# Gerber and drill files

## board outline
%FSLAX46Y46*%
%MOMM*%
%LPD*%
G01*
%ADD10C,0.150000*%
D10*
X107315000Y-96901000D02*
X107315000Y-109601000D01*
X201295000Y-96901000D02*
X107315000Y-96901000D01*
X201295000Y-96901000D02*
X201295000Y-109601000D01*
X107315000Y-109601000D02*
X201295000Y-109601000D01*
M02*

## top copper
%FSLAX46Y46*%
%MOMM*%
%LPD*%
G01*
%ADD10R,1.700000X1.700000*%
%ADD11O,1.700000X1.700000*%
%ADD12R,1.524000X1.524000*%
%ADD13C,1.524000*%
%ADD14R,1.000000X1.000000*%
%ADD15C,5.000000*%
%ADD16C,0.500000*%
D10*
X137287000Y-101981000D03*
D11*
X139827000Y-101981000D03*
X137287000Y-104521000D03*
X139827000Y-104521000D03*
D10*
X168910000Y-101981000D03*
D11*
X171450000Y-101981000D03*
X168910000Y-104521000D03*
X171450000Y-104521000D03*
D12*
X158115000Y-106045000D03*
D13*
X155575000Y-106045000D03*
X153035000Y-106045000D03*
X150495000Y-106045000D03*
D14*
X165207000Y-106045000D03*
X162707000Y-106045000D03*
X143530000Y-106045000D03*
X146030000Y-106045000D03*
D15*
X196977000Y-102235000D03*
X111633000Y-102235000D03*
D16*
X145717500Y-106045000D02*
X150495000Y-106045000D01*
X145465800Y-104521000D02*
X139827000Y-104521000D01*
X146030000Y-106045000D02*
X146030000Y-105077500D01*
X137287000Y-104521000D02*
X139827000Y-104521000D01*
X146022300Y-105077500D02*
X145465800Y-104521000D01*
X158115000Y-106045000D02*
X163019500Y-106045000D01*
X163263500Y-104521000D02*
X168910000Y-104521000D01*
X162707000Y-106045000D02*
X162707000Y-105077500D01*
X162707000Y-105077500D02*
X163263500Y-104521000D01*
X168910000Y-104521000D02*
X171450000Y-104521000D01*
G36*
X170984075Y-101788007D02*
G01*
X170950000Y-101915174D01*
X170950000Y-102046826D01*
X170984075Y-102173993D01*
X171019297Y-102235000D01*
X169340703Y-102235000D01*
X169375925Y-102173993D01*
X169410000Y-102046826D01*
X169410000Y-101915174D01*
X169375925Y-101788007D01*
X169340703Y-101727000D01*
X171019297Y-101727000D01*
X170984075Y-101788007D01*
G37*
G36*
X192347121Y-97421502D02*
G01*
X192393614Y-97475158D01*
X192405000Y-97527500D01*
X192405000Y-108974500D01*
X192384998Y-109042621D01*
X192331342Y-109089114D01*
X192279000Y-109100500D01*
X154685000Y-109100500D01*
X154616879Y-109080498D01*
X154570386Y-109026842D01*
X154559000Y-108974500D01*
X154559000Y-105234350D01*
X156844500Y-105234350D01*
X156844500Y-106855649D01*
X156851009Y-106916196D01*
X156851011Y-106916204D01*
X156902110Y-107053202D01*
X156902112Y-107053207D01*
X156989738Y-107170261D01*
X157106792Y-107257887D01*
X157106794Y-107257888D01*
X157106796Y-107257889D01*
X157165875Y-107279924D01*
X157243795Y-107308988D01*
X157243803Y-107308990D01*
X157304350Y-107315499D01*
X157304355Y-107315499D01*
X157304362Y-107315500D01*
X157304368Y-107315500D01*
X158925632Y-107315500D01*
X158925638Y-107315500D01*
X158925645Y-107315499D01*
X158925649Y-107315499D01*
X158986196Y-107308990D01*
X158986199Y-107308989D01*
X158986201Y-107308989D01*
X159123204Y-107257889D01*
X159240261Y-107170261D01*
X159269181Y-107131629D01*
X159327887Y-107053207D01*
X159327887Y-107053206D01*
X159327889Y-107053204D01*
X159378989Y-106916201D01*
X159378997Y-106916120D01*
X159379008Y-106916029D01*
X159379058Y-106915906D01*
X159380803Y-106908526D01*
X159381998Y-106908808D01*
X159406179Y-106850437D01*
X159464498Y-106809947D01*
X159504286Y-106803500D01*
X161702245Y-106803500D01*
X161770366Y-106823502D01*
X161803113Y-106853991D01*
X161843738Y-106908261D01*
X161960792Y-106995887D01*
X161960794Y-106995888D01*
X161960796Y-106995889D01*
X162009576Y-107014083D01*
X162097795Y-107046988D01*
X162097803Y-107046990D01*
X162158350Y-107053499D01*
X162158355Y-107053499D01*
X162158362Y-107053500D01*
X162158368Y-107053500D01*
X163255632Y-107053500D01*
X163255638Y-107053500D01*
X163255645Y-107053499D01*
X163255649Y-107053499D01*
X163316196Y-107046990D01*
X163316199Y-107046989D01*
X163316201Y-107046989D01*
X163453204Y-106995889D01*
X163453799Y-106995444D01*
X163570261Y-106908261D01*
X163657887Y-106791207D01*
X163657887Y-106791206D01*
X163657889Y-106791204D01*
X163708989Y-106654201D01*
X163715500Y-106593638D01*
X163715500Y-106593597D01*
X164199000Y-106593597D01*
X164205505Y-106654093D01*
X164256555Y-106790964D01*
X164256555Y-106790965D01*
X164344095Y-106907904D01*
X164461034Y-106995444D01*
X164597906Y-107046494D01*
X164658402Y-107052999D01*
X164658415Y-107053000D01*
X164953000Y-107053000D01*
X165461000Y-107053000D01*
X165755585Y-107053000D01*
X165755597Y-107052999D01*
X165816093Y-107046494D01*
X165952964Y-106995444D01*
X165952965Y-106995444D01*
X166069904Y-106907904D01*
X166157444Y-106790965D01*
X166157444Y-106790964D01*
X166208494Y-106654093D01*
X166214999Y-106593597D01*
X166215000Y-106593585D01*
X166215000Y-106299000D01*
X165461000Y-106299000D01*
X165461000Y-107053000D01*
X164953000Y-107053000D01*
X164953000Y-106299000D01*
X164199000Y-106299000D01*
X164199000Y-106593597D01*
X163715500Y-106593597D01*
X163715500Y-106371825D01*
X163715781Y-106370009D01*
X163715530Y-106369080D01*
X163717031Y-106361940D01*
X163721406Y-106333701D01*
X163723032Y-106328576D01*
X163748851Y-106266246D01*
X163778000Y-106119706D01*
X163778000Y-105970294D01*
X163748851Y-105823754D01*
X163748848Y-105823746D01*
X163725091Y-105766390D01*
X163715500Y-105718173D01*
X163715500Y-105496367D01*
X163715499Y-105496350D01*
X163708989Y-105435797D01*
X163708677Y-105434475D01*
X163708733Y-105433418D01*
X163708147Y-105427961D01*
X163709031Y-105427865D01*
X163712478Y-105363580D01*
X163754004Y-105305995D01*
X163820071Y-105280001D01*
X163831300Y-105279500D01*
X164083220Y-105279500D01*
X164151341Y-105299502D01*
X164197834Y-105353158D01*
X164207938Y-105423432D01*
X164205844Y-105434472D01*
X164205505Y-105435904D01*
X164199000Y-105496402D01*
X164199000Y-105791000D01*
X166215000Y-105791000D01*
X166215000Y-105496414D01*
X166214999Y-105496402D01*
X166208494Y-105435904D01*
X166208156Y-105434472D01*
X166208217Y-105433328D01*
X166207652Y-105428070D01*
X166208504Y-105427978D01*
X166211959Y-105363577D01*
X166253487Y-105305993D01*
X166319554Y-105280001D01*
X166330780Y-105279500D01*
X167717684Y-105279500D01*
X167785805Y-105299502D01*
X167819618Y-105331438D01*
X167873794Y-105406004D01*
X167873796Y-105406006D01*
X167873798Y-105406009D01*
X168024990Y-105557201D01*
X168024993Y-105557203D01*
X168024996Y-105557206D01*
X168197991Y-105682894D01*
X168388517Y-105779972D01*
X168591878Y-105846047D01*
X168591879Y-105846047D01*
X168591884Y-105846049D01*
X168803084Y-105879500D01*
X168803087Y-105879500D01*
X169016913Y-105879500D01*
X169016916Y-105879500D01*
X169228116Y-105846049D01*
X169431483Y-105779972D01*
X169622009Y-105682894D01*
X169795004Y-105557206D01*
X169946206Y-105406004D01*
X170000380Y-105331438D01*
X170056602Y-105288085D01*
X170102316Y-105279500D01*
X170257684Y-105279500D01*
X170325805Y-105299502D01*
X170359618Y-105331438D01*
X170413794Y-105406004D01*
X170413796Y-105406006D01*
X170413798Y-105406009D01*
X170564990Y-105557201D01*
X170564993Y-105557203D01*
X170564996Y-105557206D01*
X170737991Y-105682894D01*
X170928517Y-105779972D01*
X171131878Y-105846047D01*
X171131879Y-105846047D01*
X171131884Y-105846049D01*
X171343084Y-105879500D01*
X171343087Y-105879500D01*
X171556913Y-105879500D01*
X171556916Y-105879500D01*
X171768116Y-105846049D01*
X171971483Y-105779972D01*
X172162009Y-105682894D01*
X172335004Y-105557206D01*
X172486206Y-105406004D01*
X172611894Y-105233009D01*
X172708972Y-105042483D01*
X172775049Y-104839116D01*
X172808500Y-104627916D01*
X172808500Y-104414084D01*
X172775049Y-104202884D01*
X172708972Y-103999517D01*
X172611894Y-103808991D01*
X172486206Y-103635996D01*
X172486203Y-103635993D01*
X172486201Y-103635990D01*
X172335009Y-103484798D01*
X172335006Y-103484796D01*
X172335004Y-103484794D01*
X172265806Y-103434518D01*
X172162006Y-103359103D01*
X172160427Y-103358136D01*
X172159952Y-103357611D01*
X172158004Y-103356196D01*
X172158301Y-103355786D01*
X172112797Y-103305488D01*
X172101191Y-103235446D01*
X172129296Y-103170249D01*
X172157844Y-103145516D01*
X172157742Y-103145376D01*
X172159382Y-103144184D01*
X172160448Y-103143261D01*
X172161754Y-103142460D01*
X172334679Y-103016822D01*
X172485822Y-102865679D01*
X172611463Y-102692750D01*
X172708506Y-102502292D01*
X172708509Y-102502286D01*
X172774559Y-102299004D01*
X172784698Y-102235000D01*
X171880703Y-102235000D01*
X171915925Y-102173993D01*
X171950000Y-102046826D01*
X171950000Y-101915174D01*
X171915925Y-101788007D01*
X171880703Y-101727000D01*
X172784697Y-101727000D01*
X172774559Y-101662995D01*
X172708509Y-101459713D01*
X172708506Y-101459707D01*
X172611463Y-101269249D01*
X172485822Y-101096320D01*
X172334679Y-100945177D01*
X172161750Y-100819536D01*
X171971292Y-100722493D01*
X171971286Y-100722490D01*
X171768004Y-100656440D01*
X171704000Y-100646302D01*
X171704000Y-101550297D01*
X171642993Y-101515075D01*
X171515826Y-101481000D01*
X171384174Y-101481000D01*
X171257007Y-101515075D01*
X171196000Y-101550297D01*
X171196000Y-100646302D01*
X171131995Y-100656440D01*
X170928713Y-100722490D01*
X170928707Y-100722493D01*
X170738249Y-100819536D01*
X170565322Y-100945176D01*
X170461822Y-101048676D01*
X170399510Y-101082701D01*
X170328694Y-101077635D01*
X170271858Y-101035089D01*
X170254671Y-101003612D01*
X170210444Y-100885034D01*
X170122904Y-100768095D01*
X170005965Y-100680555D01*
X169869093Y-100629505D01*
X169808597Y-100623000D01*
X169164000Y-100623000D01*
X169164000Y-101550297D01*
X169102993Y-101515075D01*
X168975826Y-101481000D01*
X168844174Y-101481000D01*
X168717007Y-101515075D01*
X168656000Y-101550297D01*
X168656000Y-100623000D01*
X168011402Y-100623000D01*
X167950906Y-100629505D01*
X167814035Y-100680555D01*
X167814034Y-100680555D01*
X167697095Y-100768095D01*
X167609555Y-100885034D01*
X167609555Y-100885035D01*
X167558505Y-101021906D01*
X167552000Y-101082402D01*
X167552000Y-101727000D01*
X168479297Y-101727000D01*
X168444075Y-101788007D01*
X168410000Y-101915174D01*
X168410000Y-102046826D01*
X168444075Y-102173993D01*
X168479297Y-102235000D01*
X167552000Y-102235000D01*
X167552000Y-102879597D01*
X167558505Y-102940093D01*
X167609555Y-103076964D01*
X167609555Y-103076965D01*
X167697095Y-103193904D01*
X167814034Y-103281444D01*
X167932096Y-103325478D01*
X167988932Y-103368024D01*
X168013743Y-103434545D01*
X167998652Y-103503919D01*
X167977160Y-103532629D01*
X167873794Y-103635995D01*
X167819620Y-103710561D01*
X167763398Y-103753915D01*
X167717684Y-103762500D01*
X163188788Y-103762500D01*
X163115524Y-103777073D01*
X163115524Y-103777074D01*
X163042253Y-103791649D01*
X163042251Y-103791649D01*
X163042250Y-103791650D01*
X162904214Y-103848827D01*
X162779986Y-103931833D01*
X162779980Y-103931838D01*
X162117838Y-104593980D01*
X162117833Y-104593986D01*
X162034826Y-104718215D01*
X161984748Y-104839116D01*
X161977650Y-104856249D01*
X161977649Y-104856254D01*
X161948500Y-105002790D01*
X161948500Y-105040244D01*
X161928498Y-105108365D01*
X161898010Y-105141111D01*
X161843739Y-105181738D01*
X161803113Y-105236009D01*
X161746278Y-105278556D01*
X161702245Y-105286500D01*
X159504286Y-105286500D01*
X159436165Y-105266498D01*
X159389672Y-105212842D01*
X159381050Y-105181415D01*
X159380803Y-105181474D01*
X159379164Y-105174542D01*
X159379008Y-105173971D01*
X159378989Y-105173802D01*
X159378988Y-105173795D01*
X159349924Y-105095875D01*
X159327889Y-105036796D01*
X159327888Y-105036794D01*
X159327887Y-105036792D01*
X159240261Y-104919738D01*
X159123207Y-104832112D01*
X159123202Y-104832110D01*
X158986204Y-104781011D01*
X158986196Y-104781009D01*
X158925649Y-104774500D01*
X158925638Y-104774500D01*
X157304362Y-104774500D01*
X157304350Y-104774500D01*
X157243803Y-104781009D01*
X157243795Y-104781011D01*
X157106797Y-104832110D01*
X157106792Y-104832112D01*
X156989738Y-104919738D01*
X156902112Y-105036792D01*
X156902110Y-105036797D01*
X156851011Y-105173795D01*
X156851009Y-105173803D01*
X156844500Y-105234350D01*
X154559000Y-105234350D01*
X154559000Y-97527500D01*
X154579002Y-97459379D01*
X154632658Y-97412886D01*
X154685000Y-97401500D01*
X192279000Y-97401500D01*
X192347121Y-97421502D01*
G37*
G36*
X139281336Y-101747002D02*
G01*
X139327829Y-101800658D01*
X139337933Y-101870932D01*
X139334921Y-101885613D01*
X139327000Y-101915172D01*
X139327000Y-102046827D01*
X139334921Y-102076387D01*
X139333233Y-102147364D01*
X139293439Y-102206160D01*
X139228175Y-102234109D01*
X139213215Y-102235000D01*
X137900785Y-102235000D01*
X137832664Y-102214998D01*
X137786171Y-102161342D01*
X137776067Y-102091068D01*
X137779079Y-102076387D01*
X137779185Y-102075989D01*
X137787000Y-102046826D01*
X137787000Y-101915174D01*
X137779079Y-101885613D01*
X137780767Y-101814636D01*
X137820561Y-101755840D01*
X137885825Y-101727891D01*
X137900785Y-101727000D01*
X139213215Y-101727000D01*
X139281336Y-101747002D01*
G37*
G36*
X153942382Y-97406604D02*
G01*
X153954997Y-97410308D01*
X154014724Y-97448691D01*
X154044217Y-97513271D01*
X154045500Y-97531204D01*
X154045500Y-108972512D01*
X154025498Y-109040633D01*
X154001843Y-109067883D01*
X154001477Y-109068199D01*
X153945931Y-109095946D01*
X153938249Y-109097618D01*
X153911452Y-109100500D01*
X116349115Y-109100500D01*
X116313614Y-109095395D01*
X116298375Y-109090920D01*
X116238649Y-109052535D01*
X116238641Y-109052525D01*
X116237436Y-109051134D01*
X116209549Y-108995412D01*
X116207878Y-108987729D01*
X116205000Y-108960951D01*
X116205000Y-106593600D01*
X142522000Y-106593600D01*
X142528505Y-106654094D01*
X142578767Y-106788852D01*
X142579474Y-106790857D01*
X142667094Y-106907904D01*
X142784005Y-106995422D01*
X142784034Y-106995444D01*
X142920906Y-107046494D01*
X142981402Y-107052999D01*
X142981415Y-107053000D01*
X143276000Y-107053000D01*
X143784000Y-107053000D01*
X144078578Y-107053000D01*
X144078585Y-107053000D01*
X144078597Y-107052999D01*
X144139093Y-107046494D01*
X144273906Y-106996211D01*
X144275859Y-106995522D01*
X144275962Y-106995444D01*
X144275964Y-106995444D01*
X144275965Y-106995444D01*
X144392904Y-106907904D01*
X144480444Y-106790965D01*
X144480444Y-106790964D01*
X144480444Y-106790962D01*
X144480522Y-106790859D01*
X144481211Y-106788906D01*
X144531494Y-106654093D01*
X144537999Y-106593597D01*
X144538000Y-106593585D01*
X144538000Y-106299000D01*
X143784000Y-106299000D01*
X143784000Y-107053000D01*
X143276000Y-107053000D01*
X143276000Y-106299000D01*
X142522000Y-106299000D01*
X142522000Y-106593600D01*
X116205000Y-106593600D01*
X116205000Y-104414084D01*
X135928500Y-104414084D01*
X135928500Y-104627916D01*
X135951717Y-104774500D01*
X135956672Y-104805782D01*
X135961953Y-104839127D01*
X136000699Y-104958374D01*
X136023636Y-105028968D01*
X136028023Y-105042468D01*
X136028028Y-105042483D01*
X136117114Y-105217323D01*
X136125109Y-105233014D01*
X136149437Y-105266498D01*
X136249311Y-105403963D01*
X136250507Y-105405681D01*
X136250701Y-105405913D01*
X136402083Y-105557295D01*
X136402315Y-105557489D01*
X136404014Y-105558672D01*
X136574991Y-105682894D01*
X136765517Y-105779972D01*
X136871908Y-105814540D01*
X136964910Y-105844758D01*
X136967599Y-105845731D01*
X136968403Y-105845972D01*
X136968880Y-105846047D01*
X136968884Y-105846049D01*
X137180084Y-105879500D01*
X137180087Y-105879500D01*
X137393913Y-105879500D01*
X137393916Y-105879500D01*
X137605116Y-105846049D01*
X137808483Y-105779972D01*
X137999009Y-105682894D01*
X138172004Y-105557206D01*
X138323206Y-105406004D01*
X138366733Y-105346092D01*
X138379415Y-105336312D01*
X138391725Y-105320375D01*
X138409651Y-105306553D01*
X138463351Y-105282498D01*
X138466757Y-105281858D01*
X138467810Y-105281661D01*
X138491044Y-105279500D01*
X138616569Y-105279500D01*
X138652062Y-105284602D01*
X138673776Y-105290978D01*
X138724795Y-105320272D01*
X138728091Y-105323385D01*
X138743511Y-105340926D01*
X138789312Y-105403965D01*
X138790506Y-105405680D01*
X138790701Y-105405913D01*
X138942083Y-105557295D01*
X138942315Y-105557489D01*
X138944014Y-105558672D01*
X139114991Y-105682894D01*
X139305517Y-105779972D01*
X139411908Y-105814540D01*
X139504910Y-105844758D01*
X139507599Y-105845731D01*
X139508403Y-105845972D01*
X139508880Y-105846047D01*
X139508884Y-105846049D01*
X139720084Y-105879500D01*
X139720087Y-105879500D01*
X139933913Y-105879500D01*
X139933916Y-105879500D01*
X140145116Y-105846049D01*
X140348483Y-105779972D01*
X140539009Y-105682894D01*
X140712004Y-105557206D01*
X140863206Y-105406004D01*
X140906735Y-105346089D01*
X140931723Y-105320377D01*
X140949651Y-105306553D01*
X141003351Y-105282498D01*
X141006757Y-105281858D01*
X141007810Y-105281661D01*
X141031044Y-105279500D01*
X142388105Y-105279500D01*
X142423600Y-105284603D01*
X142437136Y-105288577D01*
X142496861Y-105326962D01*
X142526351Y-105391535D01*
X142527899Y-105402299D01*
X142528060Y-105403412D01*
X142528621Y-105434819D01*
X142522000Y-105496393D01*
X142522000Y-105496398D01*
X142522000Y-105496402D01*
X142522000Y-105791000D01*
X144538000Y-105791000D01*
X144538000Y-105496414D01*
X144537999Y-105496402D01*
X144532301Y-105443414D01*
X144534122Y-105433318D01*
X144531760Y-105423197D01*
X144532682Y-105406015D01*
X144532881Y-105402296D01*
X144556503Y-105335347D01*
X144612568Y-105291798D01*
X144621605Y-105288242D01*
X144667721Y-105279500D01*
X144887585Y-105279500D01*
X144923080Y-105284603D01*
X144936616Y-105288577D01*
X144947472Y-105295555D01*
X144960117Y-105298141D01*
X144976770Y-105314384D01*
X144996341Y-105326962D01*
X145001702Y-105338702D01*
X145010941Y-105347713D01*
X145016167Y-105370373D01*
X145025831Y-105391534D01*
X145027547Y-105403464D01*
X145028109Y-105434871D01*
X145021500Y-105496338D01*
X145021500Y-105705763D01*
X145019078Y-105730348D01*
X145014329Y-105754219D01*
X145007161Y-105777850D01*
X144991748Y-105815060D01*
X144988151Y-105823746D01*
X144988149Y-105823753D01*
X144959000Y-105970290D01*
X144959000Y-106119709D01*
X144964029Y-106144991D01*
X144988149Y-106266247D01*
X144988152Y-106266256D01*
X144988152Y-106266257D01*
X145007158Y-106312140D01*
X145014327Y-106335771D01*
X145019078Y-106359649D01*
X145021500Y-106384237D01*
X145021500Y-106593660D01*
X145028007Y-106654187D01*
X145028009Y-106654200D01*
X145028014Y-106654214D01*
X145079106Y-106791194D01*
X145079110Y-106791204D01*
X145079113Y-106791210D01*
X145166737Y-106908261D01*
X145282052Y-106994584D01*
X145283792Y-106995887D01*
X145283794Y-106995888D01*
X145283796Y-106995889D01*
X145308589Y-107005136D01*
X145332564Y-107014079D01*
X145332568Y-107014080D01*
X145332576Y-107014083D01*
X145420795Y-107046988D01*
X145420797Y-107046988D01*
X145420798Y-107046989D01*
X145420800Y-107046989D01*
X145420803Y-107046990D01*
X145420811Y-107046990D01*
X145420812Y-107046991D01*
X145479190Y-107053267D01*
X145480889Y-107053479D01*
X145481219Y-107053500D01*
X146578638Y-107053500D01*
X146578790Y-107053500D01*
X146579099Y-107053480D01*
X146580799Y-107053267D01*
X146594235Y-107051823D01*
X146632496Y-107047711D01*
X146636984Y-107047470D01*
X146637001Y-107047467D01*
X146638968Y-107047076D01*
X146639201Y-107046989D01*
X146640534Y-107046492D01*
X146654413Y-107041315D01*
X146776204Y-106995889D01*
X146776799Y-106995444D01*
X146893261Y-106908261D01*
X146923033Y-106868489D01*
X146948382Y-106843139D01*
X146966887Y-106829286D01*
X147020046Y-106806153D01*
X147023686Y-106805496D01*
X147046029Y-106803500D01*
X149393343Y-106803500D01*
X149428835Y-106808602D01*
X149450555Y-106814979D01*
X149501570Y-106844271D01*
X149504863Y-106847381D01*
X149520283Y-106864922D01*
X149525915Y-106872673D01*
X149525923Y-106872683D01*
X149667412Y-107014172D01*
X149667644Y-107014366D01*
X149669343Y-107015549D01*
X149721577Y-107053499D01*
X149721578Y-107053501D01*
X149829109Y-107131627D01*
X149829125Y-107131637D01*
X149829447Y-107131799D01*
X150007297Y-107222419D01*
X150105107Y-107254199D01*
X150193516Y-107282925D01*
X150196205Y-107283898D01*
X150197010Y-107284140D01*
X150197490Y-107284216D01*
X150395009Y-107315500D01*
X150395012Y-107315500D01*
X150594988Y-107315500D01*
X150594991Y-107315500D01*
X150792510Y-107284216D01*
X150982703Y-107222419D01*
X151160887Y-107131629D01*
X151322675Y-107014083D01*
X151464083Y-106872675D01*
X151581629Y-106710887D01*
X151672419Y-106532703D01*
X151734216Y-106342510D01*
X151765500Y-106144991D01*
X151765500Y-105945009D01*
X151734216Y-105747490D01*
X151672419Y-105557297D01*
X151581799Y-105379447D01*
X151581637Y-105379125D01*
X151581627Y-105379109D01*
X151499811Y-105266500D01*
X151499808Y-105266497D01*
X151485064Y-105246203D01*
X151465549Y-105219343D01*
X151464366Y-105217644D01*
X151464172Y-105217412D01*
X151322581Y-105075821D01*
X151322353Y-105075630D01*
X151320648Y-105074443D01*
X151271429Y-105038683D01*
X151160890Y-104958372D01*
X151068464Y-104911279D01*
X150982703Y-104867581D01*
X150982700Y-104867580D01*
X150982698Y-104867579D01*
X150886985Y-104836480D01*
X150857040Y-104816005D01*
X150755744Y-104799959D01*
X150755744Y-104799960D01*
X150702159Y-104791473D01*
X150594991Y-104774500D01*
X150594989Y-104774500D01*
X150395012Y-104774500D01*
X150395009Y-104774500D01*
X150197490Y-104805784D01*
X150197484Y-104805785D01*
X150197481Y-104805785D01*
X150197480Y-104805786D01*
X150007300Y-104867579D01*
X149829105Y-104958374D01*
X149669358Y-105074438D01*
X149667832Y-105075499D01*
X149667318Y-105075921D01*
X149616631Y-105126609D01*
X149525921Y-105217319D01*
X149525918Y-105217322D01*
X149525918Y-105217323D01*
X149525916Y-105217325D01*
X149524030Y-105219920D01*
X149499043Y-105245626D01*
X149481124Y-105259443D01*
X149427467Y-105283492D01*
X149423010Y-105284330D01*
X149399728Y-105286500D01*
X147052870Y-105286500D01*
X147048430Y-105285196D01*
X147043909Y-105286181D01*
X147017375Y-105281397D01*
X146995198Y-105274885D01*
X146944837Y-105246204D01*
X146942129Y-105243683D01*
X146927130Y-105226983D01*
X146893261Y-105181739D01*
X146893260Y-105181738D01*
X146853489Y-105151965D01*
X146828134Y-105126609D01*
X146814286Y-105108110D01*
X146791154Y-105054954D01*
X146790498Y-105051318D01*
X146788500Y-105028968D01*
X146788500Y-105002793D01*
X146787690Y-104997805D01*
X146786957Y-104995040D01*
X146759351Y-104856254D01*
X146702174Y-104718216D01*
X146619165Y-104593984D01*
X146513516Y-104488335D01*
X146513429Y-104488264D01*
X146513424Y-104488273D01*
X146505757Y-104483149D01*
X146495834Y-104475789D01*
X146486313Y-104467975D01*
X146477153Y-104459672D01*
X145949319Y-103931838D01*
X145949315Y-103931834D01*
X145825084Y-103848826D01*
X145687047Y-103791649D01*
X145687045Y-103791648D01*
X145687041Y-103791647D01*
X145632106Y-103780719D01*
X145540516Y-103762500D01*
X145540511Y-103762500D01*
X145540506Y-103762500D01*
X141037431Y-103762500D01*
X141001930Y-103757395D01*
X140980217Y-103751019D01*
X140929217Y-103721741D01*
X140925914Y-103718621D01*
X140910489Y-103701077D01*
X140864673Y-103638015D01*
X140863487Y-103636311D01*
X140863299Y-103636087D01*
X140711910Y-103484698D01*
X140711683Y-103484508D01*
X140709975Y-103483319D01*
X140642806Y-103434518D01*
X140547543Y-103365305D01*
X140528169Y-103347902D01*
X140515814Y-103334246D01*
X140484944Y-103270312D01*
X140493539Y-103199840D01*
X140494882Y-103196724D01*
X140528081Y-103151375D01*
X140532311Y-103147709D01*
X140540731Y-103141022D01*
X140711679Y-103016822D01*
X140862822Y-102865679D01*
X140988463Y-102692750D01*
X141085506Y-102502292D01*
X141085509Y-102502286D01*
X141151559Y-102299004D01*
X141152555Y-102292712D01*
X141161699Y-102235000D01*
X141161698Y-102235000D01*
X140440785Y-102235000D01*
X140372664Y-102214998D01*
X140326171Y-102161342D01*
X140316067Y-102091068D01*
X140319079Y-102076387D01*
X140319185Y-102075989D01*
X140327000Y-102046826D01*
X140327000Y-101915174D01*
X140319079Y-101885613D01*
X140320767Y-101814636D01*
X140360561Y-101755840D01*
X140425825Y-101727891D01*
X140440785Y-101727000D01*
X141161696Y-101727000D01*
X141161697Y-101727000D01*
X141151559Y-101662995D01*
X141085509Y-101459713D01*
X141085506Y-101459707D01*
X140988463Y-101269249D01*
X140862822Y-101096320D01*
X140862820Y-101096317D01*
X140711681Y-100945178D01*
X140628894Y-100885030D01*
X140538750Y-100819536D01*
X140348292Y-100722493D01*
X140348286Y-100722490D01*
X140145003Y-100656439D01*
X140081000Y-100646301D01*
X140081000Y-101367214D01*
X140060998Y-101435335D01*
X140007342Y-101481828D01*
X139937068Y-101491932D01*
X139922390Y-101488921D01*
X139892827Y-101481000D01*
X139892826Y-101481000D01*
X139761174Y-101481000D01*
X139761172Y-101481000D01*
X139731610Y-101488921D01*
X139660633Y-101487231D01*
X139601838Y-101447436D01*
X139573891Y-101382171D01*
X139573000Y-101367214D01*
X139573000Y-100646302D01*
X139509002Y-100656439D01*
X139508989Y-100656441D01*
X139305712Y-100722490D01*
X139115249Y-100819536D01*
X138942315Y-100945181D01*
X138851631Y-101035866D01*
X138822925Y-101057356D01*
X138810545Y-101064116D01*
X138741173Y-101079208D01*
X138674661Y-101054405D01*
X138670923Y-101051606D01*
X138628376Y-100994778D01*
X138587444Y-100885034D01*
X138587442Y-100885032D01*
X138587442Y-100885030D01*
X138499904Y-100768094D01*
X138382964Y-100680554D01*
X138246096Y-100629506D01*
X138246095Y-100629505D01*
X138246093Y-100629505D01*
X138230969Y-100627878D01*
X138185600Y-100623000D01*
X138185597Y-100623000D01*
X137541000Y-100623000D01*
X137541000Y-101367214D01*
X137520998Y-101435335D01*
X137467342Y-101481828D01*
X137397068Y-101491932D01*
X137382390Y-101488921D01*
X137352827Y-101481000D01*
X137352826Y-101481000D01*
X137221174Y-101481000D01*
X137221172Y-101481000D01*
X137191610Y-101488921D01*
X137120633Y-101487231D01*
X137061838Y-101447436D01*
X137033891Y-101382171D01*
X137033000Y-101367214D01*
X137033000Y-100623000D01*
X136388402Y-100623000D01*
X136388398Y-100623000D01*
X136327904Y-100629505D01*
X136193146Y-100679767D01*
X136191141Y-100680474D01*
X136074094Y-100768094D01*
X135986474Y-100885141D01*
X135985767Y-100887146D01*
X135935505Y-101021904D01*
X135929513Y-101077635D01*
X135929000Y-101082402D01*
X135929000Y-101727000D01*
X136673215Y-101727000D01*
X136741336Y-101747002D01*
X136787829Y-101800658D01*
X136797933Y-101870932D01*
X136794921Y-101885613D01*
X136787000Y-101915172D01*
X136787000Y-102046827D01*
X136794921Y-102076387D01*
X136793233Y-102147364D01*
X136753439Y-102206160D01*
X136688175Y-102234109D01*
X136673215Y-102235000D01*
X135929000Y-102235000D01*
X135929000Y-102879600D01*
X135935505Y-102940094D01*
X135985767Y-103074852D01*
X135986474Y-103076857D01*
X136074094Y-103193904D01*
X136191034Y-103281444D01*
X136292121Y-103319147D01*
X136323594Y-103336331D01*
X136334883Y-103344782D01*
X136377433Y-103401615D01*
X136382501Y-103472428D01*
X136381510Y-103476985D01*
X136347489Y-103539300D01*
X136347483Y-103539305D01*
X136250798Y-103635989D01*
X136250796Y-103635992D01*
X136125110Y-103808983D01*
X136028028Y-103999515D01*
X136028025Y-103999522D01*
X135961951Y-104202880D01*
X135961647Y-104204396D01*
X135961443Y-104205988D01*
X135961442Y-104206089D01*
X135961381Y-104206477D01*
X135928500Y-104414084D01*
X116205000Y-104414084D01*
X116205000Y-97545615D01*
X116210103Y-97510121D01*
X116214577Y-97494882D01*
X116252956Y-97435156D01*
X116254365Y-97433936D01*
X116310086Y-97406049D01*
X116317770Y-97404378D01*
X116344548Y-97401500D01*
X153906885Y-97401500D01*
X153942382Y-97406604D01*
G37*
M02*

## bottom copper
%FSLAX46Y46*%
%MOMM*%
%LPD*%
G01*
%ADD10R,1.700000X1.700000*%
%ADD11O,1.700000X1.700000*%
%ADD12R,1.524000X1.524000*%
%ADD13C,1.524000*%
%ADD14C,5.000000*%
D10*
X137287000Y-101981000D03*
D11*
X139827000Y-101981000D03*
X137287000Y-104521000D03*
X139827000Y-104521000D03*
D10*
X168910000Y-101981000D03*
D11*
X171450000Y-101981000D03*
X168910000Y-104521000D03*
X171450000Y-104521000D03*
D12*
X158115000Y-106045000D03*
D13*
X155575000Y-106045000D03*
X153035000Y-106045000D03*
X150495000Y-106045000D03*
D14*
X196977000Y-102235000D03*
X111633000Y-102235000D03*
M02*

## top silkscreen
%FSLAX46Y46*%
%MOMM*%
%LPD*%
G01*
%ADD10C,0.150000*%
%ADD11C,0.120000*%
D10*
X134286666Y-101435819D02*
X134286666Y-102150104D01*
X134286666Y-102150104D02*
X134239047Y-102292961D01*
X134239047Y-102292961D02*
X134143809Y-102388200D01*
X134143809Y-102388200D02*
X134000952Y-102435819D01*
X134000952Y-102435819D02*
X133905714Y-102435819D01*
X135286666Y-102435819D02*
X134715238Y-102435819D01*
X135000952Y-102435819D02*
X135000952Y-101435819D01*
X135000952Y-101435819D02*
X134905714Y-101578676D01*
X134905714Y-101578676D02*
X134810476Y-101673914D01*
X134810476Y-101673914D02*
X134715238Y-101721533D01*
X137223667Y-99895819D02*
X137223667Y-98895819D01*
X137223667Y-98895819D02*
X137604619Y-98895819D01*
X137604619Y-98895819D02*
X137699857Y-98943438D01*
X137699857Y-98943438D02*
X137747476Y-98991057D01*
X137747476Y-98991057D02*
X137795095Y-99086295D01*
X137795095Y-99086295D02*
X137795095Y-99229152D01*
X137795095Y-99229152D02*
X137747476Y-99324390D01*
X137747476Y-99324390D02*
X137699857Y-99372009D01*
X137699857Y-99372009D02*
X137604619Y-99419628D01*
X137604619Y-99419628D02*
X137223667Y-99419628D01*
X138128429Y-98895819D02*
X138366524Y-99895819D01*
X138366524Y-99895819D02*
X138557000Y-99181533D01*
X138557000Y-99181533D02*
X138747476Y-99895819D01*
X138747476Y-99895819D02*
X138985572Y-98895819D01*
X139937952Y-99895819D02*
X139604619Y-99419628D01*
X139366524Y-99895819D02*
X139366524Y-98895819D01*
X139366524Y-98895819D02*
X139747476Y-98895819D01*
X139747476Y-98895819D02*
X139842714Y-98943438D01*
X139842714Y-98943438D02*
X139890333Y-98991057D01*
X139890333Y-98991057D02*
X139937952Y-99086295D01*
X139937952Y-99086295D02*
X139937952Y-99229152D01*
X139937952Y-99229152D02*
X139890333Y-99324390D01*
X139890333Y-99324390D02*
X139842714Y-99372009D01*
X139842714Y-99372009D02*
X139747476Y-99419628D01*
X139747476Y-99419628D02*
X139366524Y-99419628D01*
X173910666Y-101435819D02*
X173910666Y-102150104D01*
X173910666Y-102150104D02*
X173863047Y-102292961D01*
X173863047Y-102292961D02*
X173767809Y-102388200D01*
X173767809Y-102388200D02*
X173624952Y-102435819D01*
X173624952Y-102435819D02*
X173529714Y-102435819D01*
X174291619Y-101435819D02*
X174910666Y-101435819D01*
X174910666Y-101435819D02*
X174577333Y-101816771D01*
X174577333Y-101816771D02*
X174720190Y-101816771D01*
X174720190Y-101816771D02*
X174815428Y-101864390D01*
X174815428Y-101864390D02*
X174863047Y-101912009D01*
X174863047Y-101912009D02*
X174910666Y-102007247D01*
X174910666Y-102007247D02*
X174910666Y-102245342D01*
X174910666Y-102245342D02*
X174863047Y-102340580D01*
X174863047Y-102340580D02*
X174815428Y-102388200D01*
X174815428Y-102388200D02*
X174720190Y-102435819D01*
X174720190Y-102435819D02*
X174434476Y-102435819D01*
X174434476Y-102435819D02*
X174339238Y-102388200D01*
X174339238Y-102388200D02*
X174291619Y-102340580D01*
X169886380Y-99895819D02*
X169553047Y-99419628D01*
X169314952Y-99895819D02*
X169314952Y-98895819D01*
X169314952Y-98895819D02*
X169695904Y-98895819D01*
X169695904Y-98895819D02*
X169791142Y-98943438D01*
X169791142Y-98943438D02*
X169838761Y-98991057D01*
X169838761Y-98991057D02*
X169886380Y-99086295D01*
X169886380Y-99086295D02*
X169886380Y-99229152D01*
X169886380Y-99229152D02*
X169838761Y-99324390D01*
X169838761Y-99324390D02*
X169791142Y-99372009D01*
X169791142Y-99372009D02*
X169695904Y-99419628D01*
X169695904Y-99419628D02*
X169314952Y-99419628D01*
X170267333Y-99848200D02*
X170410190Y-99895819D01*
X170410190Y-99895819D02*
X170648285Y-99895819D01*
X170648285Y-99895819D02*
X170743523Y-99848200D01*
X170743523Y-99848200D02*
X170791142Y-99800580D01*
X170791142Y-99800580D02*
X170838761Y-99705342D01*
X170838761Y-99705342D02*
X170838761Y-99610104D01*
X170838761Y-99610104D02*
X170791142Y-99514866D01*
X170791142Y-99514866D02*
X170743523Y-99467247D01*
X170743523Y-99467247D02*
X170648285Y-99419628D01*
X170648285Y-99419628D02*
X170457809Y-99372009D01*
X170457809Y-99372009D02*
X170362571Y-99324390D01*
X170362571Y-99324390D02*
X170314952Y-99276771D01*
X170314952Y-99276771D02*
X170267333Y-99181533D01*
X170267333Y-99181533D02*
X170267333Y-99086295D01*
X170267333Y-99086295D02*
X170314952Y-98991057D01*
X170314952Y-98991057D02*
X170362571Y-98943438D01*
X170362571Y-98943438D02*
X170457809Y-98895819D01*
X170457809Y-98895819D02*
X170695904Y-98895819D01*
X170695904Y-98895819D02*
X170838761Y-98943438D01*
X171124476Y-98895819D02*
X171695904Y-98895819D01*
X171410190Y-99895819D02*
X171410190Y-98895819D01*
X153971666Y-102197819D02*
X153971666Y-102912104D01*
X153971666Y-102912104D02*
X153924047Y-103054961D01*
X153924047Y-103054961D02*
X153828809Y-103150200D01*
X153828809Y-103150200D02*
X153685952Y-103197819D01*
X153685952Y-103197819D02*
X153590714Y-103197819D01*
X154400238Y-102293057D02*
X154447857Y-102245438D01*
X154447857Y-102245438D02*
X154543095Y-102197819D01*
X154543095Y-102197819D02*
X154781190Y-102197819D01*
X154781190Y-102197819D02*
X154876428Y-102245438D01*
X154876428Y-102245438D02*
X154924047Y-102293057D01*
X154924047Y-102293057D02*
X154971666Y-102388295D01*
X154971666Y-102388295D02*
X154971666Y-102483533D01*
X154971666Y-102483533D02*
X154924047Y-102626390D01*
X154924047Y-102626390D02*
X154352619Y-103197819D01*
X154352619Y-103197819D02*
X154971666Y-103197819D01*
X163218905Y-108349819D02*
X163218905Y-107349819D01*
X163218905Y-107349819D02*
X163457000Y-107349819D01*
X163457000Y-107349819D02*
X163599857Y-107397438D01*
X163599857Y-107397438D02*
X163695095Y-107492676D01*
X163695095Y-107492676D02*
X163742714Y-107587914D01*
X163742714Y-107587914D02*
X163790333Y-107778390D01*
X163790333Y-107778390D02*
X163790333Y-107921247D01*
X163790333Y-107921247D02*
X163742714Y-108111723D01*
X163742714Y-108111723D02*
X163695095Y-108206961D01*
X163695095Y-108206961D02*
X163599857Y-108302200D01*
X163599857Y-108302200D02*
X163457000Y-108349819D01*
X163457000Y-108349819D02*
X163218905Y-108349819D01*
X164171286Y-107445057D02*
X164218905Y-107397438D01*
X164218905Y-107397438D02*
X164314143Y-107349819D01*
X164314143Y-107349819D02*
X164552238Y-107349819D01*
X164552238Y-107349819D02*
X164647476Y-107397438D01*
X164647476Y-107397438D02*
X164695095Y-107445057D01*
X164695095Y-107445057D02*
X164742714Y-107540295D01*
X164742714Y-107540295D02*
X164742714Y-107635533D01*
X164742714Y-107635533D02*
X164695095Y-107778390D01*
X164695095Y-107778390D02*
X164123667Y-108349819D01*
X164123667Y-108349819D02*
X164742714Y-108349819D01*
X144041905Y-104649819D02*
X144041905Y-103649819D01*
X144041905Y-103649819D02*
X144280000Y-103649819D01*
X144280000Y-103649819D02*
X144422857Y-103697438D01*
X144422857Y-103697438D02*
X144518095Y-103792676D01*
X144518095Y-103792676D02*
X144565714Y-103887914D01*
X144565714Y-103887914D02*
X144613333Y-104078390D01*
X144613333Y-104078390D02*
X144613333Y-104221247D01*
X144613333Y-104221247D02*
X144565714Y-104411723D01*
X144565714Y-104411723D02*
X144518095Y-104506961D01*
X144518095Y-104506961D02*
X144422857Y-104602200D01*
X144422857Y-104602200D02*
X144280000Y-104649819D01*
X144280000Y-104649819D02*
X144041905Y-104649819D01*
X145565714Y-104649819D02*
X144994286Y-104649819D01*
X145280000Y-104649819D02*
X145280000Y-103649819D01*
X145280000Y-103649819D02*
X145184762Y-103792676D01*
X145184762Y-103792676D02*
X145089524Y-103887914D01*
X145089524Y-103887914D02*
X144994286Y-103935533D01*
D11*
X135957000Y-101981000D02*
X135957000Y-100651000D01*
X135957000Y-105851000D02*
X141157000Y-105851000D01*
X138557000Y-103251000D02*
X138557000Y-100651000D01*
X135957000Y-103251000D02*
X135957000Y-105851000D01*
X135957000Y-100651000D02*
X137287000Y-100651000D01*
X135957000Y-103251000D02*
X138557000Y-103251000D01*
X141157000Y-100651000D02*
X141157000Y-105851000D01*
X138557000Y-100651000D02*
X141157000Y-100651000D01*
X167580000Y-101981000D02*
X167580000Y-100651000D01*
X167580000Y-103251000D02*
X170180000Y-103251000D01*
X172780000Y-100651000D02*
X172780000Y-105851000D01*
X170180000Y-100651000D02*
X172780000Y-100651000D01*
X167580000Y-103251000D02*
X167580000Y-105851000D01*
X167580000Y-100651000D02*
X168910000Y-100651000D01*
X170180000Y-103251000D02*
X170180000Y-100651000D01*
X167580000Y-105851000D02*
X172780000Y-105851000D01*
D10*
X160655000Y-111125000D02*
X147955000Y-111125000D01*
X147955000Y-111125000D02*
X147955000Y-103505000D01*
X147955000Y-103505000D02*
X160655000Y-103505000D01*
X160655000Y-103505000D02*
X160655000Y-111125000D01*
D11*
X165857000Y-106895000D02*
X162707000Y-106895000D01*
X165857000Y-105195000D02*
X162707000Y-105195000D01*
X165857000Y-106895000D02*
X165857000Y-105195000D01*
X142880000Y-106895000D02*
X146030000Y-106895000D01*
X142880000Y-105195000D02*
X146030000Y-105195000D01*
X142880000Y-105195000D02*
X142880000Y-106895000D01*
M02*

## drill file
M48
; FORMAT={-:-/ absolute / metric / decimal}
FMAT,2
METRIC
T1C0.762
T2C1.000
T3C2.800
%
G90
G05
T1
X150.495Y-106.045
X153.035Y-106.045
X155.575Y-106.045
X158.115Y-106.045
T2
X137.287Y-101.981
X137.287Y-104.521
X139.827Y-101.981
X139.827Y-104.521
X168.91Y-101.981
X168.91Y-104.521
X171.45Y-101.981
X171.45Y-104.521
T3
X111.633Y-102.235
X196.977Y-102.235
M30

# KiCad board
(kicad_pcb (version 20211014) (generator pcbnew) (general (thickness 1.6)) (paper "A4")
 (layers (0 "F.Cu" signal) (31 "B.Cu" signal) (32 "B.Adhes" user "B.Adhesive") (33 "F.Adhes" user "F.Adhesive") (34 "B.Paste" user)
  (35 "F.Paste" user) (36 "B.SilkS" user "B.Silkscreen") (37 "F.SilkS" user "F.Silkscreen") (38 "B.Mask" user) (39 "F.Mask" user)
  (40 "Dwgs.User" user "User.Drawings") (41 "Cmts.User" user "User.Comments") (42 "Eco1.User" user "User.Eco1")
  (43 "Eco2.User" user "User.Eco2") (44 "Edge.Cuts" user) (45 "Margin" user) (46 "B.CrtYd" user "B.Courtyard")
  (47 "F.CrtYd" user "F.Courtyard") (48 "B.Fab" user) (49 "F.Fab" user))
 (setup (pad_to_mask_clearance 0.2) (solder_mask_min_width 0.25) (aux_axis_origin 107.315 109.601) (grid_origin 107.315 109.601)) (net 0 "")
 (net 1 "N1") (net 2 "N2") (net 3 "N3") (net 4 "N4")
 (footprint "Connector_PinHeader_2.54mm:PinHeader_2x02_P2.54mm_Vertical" (layer "F.Cu") (at 137.287 101.981)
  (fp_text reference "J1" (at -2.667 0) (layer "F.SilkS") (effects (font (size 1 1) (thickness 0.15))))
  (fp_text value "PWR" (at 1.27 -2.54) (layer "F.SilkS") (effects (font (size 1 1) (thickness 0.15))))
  (fp_line (start -1.33 0) (end -1.33 -1.33) (layer "F.SilkS") (width 0.12))
  (fp_line (start -1.33 3.87) (end 3.87 3.87) (layer "F.SilkS") (width 0.12))
  (fp_line (start 1.27 1.27) (end 1.27 -1.33) (layer "F.SilkS") (width 0.12))
  (fp_line (start -1.33 1.27) (end -1.33 3.87) (layer "F.SilkS") (width 0.12))
  (fp_line (start -1.33 -1.33) (end 0 -1.33) (layer "F.SilkS") (width 0.12))
  (fp_line (start -1.33 1.27) (end 1.27 1.27) (layer "F.SilkS") (width 0.12))
  (fp_line (start 3.87 -1.33) (end 3.87 3.87) (layer "F.SilkS") (width 0.12))
  (fp_line (start 1.27 -1.33) (end 3.87 -1.33) (layer "F.SilkS") (width 0.12))
  (pad "1" thru_hole rect locked (at 0 0) (size 1.7 1.7) (drill 1) (layers *.Cu *.Mask) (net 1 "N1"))
  (pad "2" thru_hole oval locked (at 2.54 0) (size 1.7 1.7) (drill 1) (layers *.Cu *.Mask) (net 1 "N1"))
  (pad "3" thru_hole oval locked (at 0 2.54) (size 1.7 1.7) (drill 1) (layers *.Cu *.Mask) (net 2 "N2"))
  (pad "4" thru_hole oval locked (at 2.54 2.54) (size 1.7 1.7) (drill 1) (layers *.Cu *.Mask) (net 2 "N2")))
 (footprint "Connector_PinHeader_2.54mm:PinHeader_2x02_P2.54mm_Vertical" (layer "F.Cu") (at 168.91 101.981)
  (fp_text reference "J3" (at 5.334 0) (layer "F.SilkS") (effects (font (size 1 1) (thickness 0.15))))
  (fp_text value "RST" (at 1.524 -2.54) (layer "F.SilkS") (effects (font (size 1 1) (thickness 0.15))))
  (fp_line (start -1.33 0) (end -1.33 -1.33) (layer "F.SilkS") (width 0.12))
  (fp_line (start -1.33 1.27) (end 1.27 1.27) (layer "F.SilkS") (width 0.12))
  (fp_line (start 3.87 -1.33) (end 3.87 3.87) (layer "F.SilkS") (width 0.12))
  (fp_line (start 1.27 -1.33) (end 3.87 -1.33) (layer "F.SilkS") (width 0.12))
  (fp_line (start -1.33 1.27) (end -1.33 3.87) (layer "F.SilkS") (width 0.12))
  (fp_line (start -1.33 -1.33) (end 0 -1.33) (layer "F.SilkS") (width 0.12))
  (fp_line (start 1.27 1.27) (end 1.27 -1.33) (layer "F.SilkS") (width 0.12))
  (fp_line (start -1.33 3.87) (end 3.87 3.87) (layer "F.SilkS") (width 0.12))
  (pad "1" thru_hole rect locked (at 0 0) (size 1.7 1.7) (drill 1) (layers *.Cu *.Mask) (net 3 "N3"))
  (pad "2" thru_hole oval locked (at 2.54 0) (size 1.7 1.7) (drill 1) (layers *.Cu *.Mask) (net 3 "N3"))
  (pad "3" thru_hole oval locked (at 0 2.54) (size 1.7 1.7) (drill 1) (layers *.Cu *.Mask) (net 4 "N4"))
  (pad "4" thru_hole oval locked (at 2.54 2.54) (size 1.7 1.7) (drill 1) (layers *.Cu *.Mask) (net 4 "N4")))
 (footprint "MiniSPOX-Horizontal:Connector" (layer "F.Cu") (at 147.955 111.125)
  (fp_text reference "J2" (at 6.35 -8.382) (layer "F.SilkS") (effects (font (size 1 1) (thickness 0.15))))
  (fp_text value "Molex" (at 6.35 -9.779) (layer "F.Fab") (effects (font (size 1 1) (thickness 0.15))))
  (fp_line (start 12.7 0) (end 0 0) (layer "F.SilkS") (width 0.15))
  (fp_line (start 0 0) (end 0 -7.62) (layer "F.SilkS") (width 0.15))
  (fp_line (start 0 -7.62) (end 12.7 -7.62) (layer "F.SilkS") (width 0.15))
  (fp_line (start 12.7 -7.62) (end 12.7 0) (layer "F.SilkS") (width 0.15))
  (pad "1" thru_hole rect locked (at 10.16 -5.08) (size 1.524 1.524) (drill 0.762) (layers *.Cu *.Mask) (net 4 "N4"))
  (pad "2" thru_hole circle locked (at 7.62 -5.08) (size 1.524 1.524) (drill 0.762) (layers *.Cu *.Mask) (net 3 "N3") (zone_connect 2))
  (pad "3" thru_hole circle locked (at 5.08 -5.08) (size 1.524 1.524) (drill 0.762) (layers *.Cu *.Mask) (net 1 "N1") (zone_connect 2))
  (pad "4" thru_hole circle locked (at 2.54 -5.08) (size 1.524 1.524) (drill 0.762) (layers *.Cu *.Mask) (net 2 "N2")))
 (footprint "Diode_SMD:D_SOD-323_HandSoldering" (layer "F.Cu") (at 163.957 106.045 180)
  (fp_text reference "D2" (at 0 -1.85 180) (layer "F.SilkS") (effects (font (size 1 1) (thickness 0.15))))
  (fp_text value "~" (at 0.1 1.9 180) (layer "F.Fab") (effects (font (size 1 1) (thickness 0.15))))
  (fp_line (start -1.9 -0.85) (end 1.25 -0.85) (layer "F.SilkS") (width 0.12))
  (fp_line (start -1.9 0.85) (end 1.25 0.85) (layer "F.SilkS") (width 0.12))
  (fp_line (start -1.9 -0.85) (end -1.9 0.85) (layer "F.SilkS") (width 0.12))
  (pad "1" smd rect locked (at -1.25 0 180) (size 1 1) (layers "F.Cu" "F.Paste" "F.Mask") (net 3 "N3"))
  (pad "2" smd rect locked (at 1.25 0 180) (size 1 1) (layers "F.Cu" "F.Paste" "F.Mask") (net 4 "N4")))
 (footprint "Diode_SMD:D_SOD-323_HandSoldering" (layer "F.Cu") (at 144.78 106.045)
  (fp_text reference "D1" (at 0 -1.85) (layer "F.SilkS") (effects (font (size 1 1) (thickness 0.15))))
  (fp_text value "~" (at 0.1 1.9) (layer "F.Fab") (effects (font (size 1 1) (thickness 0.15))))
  (fp_line (start -1.9 0.85) (end 1.25 0.85) (layer "F.SilkS") (width 0.12))
  (fp_line (start -1.9 -0.85) (end 1.25 -0.85) (layer "F.SilkS") (width 0.12))
  (fp_line (start -1.9 -0.85) (end -1.9 0.85) (layer "F.SilkS") (width 0.12))
  (pad "1" smd rect locked (at -1.25 0) (size 1 1) (layers "F.Cu" "F.Paste" "F.Mask") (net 1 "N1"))
  (pad "2" smd rect locked (at 1.25 0) (size 1 1) (layers "F.Cu" "F.Paste" "F.Mask") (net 2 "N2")))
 (gr_line (start 107.315 96.901) (end 107.315 109.601) (layer "Edge.Cuts") (width 0.15))
 (gr_line (start 201.295 96.901) (end 107.315 96.901) (layer "Edge.Cuts") (width 0.15))
 (gr_line (start 201.295 96.901) (end 201.295 109.601) (layer "Edge.Cuts") (width 0.15))
 (gr_line (start 107.315 109.601) (end 201.295 109.601) (layer "Edge.Cuts") (width 0.15))
 (via (at 196.977 102.235) (size 5) (drill 2.8) (layers "F.Cu" "B.Cu") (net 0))
 (via (at 111.633 102.235) (size 5) (drill 2.8) (layers "F.Cu" "B.Cu") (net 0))
 (segment (start 145.7175 106.045) (end 150.495 106.045) (width 0.5) (layer "F.Cu") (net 2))
 (segment (start 145.4658 104.521) (end 139.827 104.521) (width 0.5) (layer "F.Cu") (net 2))
 (segment (start 146.03 106.045) (end 146.03 105.0775) (width 0.5) (layer "F.Cu") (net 2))
 (segment (start 137.287 104.521) (end 139.827 104.521) (width 0.5) (layer "F.Cu") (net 2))
 (segment (start 146.0223 105.0775) (end 145.4658 104.521) (width 0.5) (layer "F.Cu") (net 2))
 (segment (start 158.115 106.045) (end 163.0195 106.045) (width 0.5) (layer "F.Cu") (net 4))
 (segment (start 163.2635 104.521) (end 168.91 104.521) (width 0.5) (layer "F.Cu") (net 4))
 (segment (start 162.707 106.045) (end 162.707 105.0775) (width 0.5) (layer "F.Cu") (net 4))
 (segment (start 162.707 105.0775) (end 163.2635 104.521) (width 0.5) (layer "F.Cu") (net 4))
 (segment (start 168.91 104.521) (end 171.45 104.521) (width 0.5) (layer "F.Cu") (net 4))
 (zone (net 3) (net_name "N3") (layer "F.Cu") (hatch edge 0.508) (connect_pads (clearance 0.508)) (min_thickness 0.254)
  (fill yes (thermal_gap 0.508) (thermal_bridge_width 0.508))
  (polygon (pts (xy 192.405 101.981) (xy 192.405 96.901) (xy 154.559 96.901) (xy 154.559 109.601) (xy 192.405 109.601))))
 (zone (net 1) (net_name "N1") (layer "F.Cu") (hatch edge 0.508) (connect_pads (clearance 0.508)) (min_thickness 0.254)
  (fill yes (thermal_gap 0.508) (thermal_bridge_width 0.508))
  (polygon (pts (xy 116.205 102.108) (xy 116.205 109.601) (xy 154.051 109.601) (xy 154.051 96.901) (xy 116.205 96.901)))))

